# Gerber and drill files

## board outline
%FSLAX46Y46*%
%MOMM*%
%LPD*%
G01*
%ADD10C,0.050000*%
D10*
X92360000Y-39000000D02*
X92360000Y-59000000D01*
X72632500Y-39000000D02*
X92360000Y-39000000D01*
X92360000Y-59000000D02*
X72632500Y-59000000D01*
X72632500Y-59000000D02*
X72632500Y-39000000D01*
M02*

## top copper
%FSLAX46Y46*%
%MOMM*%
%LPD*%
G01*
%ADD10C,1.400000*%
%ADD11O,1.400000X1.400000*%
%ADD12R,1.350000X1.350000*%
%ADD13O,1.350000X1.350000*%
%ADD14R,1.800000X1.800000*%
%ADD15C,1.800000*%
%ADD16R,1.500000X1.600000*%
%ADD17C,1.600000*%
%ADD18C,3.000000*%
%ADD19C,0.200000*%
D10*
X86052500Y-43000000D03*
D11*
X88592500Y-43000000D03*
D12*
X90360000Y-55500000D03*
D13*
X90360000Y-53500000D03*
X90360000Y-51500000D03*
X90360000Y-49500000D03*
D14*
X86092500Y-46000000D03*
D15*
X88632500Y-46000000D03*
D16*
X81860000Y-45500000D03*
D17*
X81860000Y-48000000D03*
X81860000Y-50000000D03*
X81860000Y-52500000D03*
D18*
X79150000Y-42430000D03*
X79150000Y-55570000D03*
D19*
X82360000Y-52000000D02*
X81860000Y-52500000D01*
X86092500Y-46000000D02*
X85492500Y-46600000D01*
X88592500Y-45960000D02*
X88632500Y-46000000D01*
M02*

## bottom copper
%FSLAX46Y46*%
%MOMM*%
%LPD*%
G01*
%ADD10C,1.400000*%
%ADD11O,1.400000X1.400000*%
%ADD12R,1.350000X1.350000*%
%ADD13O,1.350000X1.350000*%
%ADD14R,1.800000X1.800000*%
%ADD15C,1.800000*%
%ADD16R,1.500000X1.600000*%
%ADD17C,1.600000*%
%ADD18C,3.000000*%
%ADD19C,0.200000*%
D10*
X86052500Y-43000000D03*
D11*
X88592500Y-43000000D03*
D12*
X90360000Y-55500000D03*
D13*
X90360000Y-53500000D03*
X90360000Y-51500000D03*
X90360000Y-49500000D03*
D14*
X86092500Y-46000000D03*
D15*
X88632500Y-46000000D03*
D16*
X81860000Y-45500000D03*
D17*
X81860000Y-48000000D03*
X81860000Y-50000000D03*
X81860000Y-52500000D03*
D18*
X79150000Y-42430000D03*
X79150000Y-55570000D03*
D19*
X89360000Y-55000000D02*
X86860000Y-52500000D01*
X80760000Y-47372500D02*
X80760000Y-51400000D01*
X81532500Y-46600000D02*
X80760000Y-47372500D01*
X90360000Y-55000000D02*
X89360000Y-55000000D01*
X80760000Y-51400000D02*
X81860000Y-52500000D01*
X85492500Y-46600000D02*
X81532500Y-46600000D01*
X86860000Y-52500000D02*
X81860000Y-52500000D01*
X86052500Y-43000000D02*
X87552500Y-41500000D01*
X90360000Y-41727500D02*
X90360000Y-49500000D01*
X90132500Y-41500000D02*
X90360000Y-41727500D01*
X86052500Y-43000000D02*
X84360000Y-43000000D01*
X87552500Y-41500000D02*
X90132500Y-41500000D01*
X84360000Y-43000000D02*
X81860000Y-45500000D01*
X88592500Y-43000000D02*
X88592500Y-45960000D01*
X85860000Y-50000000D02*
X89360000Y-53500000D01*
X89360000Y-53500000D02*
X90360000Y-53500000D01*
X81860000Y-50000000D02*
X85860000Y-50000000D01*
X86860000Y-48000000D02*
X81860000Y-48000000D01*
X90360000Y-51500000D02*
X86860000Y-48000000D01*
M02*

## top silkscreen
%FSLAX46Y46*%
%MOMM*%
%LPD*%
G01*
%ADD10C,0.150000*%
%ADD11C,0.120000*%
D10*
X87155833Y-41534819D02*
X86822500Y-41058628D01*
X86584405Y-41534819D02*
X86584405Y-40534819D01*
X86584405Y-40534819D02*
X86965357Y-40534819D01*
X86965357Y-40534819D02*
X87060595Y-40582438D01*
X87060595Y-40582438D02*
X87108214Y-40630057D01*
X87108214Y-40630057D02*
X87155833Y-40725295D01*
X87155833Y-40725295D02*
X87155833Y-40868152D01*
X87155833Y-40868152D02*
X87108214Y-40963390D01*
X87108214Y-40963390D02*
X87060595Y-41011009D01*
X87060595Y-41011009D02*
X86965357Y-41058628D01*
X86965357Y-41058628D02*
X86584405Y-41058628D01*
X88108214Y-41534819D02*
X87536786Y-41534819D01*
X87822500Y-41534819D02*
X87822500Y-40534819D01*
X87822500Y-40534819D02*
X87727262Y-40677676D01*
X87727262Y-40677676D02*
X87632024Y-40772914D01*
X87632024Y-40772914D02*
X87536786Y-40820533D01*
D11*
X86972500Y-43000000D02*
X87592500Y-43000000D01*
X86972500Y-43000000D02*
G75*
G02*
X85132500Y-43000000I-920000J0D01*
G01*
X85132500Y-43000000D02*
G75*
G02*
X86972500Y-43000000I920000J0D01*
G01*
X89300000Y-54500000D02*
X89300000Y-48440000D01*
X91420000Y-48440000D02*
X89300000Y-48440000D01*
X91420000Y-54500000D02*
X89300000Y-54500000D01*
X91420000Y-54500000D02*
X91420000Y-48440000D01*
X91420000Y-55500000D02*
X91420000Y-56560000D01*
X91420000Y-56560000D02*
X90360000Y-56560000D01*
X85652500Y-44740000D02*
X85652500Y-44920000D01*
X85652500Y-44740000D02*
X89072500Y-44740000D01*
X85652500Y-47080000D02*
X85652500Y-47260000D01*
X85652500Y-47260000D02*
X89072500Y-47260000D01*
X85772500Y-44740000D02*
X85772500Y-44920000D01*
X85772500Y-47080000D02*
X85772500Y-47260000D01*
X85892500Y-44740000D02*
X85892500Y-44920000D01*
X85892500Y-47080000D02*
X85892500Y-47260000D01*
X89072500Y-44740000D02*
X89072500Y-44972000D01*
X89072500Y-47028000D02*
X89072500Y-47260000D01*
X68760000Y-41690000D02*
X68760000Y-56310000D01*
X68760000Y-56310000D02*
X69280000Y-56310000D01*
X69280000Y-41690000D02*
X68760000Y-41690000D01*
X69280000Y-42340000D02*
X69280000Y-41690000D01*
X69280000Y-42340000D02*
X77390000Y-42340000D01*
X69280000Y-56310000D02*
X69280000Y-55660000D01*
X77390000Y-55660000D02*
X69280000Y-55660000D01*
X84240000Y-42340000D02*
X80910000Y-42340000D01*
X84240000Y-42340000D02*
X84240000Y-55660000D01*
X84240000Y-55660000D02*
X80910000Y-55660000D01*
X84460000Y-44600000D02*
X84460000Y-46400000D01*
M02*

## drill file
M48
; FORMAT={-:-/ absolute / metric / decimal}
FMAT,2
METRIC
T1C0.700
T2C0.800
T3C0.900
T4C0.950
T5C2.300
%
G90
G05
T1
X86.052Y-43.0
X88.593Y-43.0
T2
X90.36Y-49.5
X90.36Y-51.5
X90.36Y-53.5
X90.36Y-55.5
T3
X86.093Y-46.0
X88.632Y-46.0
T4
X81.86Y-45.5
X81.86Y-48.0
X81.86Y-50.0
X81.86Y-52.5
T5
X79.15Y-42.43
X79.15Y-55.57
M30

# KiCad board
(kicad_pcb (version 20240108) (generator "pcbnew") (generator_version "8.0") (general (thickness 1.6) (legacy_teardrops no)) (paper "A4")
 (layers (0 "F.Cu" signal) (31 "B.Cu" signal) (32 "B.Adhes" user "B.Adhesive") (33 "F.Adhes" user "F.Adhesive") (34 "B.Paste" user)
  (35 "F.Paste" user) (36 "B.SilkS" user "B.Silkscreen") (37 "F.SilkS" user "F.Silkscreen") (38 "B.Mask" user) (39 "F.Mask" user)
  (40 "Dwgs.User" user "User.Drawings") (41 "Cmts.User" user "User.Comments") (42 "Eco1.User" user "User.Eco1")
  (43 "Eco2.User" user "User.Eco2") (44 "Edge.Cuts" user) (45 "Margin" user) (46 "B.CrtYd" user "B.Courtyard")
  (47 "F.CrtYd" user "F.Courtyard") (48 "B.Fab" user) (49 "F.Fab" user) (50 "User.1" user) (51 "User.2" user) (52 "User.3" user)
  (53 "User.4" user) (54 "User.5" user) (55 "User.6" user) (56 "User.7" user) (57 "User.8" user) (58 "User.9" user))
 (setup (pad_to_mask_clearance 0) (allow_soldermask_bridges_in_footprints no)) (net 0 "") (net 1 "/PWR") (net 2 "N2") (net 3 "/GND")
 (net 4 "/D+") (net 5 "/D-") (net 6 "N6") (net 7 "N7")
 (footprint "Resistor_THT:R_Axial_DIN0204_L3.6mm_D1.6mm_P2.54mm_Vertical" (layer "F.Cu") (at 86.0525 43)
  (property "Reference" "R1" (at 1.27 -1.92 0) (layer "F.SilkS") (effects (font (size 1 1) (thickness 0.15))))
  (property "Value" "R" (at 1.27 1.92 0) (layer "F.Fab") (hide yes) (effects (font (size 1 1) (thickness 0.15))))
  (fp_line (start 0.92 0) (end 1.54 0) (stroke (width 0.12) (type solid)) (layer "F.SilkS"))
  (fp_circle (center 0 0) (end 0.92 0) (stroke (width 0.12) (type solid)) (fill none) (layer "F.SilkS"))
  (pad "1" thru_hole circle (at 0 0) (size 1.4 1.4) (drill 0.7) (layers "*.Cu" "*.Mask") (remove_unused_layers no) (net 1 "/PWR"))
  (pad "2" thru_hole oval (at 2.54 0) (size 1.4 1.4) (drill 0.7) (layers "*.Cu" "*.Mask") (remove_unused_layers no) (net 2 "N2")))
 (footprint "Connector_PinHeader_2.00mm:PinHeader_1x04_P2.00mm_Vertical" (layer "F.Cu") (at 90.36 55.5 180)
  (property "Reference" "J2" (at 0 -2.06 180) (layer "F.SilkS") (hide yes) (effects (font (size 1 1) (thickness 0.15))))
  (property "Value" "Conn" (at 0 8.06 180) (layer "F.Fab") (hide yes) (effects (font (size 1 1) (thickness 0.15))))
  (fp_line (start 1.06 1) (end 1.06 7.06) (stroke (width 0.12) (type solid)) (layer "F.SilkS"))
  (fp_line (start -1.06 7.06) (end 1.06 7.06) (stroke (width 0.12) (type solid)) (layer "F.SilkS"))
  (fp_line (start -1.06 1) (end 1.06 1) (stroke (width 0.12) (type solid)) (layer "F.SilkS"))
  (fp_line (start -1.06 1) (end -1.06 7.06) (stroke (width 0.12) (type solid)) (layer "F.SilkS"))
  (fp_line (start -1.06 0) (end -1.06 -1.06) (stroke (width 0.12) (type solid)) (layer "F.SilkS"))
  (fp_line (start -1.06 -1.06) (end 0 -1.06) (stroke (width 0.12) (type solid)) (layer "F.SilkS"))
  (pad "1" thru_hole rect (at 0 0 180) (size 1.35 1.35) (drill 0.8) (layers "*.Cu" "*.Mask") (remove_unused_layers no) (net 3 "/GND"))
  (pad "2" thru_hole oval (at 0 2 180) (size 1.35 1.35) (drill 0.8) (layers "*.Cu" "*.Mask") (remove_unused_layers no) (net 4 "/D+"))
  (pad "3" thru_hole oval (at 0 4 180) (size 1.35 1.35) (drill 0.8) (layers "*.Cu" "*.Mask") (remove_unused_layers no) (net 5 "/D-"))
  (pad "4" thru_hole oval (at 0 6 180) (size 1.35 1.35) (drill 0.8) (layers "*.Cu" "*.Mask") (remove_unused_layers no) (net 1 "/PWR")))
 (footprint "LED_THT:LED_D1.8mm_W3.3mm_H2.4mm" (layer "F.Cu") (at 86.0925 46)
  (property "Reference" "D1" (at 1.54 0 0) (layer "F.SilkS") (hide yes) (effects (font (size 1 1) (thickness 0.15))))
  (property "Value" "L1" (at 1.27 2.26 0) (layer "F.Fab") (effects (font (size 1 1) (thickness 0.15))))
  (fp_line (start -0.44 -1.26) (end -0.44 -1.08) (stroke (width 0.12) (type solid)) (layer "F.SilkS"))
  (fp_line (start -0.44 -1.26) (end 2.98 -1.26) (stroke (width 0.12) (type solid)) (layer "F.SilkS"))
  (fp_line (start -0.44 1.08) (end -0.44 1.26) (stroke (width 0.12) (type solid)) (layer "F.SilkS"))
  (fp_line (start -0.44 1.26) (end 2.98 1.26) (stroke (width 0.12) (type solid)) (layer "F.SilkS"))
  (fp_line (start -0.32 -1.26) (end -0.32 -1.08) (stroke (width 0.12) (type solid)) (layer "F.SilkS"))
  (fp_line (start -0.32 1.08) (end -0.32 1.26) (stroke (width 0.12) (type solid)) (layer "F.SilkS"))
  (fp_line (start -0.2 -1.26) (end -0.2 -1.08) (stroke (width 0.12) (type solid)) (layer "F.SilkS"))
  (fp_line (start -0.2 1.08) (end -0.2 1.26) (stroke (width 0.12) (type solid)) (layer "F.SilkS"))
  (fp_line (start 2.98 -1.26) (end 2.98 -1.028) (stroke (width 0.12) (type solid)) (layer "F.SilkS"))
  (fp_line (start 2.98 1.028) (end 2.98 1.26) (stroke (width 0.12) (type solid)) (layer "F.SilkS"))
  (pad "1" thru_hole rect (at 0 0) (size 1.8 1.8) (drill 0.9) (layers "*.Cu" "*.Mask") (remove_unused_layers no) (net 3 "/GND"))
  (pad "2" thru_hole circle (at 2.54 0) (size 1.8 1.8) (drill 0.9) (layers "*.Cu" "*.Mask") (remove_unused_layers no) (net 2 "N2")))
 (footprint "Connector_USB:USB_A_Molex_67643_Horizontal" (layer "F.Cu") (at 81.86 45.5 -90)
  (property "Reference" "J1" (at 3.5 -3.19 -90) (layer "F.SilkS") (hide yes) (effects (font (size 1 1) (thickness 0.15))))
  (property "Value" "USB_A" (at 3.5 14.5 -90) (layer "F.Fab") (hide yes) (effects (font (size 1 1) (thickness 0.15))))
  (fp_line (start -3.81 13.1) (end 10.81 13.1) (stroke (width 0.12) (type solid)) (layer "F.SilkS"))
  (fp_line (start 10.81 13.1) (end 10.81 12.58) (stroke (width 0.12) (type solid)) (layer "F.SilkS"))
  (fp_line (start -3.81 12.58) (end -3.81 13.1) (stroke (width 0.12) (type solid)) (layer "F.SilkS"))
  (fp_line (start -3.16 12.58) (end -3.81 12.58) (stroke (width 0.12) (type solid)) (layer "F.SilkS"))
  (fp_line (start -3.16 12.58) (end -3.16 4.47) (stroke (width 0.12) (type solid)) (layer "F.SilkS"))
  (fp_line (start 10.81 12.58) (end 10.16 12.58) (stroke (width 0.12) (type solid)) (layer "F.SilkS"))
  (fp_line (start 10.16 4.47) (end 10.16 12.58) (stroke (width 0.12) (type solid)) (layer "F.SilkS"))
  (fp_line (start -3.16 -2.38) (end -3.16 0.95) (stroke (width 0.12) (type solid)) (layer "F.SilkS"))
  (fp_line (start -3.16 -2.38) (end 10.16 -2.38) (stroke (width 0.12) (type solid)) (layer "F.SilkS"))
  (fp_line (start 10.16 -2.38) (end 10.16 0.95) (stroke (width 0.12) (type solid)) (layer "F.SilkS"))
  (fp_line (start -0.9 -2.6) (end 0.9 -2.6) (stroke (width 0.12) (type solid)) (layer "F.SilkS"))
  (pad "1" thru_hole rect (at 0 0 270) (size 1.6 1.5) (drill 0.95) (layers "*.Cu" "*.Mask") (remove_unused_layers no) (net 1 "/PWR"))
  (pad "2" thru_hole circle (at 2.5 0 270) (size 1.6 1.6) (drill 0.95) (layers "*.Cu" "*.Mask") (remove_unused_layers no) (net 5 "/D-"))
  (pad "3" thru_hole circle (at 4.5 0 270) (size 1.6 1.6) (drill 0.95) (layers "*.Cu" "*.Mask") (remove_unused_layers no) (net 4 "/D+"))
  (pad "4" thru_hole circle (at 7 0 270) (size 1.6 1.6) (drill 0.95) (layers "*.Cu" "*.Mask") (remove_unused_layers no) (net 3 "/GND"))
  (pad "5" thru_hole circle (at -3.07 2.71 270) (size 3 3) (drill 2.3) (layers "*.Cu" "*.Mask") (remove_unused_layers no) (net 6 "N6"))
  (pad "5" thru_hole circle (at 10.07 2.71 270) (size 3 3) (drill 2.3) (layers "*.Cu" "*.Mask") (remove_unused_layers no) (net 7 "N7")))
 (gr_line (start 92.36 39) (end 92.36 59) (stroke (width 0.05) (type default)) (layer "Edge.Cuts"))
 (gr_line (start 72.6325 39) (end 92.36 39) (stroke (width 0.05) (type default)) (layer "Edge.Cuts"))
 (gr_line (start 92.36 59) (end 72.6325 59) (stroke (width 0.05) (type default)) (layer "Edge.Cuts"))
 (gr_line (start 72.6325 59) (end 72.6325 39) (stroke (width 0.05) (type default)) (layer "Edge.Cuts"))
 (segment (start 82.36 52) (end 81.86 52.5) (width 0.2) (layer "F.Cu") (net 3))
 (segment (start 86.0925 46) (end 85.4925 46.6) (width 0.2) (layer "F.Cu") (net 3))
 (segment (start 89.36 55) (end 86.86 52.5) (width 0.2) (layer "B.Cu") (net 3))
 (segment (start 80.76 47.3725) (end 80.76 51.4) (width 0.2) (layer "B.Cu") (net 3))
 (segment (start 81.5325 46.6) (end 80.76 47.3725) (width 0.2) (layer "B.Cu") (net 3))
 (segment (start 90.36 55) (end 89.36 55) (width 0.2) (layer "B.Cu") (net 3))
 (segment (start 80.76 51.4) (end 81.86 52.5) (width 0.2) (layer "B.Cu") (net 3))
 (segment (start 85.4925 46.6) (end 81.5325 46.6) (width 0.2) (layer "B.Cu") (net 3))
 (segment (start 86.86 52.5) (end 81.86 52.5) (width 0.2) (layer "B.Cu") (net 3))
 (segment (start 86.0525 43) (end 87.5525 41.5) (width 0.2) (layer "B.Cu") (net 1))
 (segment (start 90.36 41.7275) (end 90.36 49.5) (width 0.2) (layer "B.Cu") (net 1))
 (segment (start 90.1325 41.5) (end 90.36 41.7275) (width 0.2) (layer "B.Cu") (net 1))
 (segment (start 86.0525 43) (end 84.36 43) (width 0.2) (layer "B.Cu") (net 1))
 (segment (start 87.5525 41.5) (end 90.1325 41.5) (width 0.2) (layer "B.Cu") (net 1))
 (segment (start 84.36 43) (end 81.86 45.5) (width 0.2) (layer "B.Cu") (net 1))
 (segment (start 88.5925 45.96) (end 88.6325 46) (width 0.2) (layer "F.Cu") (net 2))
 (segment (start 88.5925 43) (end 88.5925 45.96) (width 0.2) (layer "B.Cu") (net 2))
 (segment (start 85.86 50) (end 89.36 53.5) (width 0.2) (layer "B.Cu") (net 4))
 (segment (start 89.36 53.5) (end 90.36 53.5) (width 0.2) (layer "B.Cu") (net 4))
 (segment (start 81.86 50) (end 85.86 50) (width 0.2) (layer "B.Cu") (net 4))
 (segment (start 86.86 48) (end 81.86 48) (width 0.2) (layer "B.Cu") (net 5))
 (segment (start 90.36 51.5) (end 86.86 48) (width 0.2) (layer "B.Cu") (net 5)))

